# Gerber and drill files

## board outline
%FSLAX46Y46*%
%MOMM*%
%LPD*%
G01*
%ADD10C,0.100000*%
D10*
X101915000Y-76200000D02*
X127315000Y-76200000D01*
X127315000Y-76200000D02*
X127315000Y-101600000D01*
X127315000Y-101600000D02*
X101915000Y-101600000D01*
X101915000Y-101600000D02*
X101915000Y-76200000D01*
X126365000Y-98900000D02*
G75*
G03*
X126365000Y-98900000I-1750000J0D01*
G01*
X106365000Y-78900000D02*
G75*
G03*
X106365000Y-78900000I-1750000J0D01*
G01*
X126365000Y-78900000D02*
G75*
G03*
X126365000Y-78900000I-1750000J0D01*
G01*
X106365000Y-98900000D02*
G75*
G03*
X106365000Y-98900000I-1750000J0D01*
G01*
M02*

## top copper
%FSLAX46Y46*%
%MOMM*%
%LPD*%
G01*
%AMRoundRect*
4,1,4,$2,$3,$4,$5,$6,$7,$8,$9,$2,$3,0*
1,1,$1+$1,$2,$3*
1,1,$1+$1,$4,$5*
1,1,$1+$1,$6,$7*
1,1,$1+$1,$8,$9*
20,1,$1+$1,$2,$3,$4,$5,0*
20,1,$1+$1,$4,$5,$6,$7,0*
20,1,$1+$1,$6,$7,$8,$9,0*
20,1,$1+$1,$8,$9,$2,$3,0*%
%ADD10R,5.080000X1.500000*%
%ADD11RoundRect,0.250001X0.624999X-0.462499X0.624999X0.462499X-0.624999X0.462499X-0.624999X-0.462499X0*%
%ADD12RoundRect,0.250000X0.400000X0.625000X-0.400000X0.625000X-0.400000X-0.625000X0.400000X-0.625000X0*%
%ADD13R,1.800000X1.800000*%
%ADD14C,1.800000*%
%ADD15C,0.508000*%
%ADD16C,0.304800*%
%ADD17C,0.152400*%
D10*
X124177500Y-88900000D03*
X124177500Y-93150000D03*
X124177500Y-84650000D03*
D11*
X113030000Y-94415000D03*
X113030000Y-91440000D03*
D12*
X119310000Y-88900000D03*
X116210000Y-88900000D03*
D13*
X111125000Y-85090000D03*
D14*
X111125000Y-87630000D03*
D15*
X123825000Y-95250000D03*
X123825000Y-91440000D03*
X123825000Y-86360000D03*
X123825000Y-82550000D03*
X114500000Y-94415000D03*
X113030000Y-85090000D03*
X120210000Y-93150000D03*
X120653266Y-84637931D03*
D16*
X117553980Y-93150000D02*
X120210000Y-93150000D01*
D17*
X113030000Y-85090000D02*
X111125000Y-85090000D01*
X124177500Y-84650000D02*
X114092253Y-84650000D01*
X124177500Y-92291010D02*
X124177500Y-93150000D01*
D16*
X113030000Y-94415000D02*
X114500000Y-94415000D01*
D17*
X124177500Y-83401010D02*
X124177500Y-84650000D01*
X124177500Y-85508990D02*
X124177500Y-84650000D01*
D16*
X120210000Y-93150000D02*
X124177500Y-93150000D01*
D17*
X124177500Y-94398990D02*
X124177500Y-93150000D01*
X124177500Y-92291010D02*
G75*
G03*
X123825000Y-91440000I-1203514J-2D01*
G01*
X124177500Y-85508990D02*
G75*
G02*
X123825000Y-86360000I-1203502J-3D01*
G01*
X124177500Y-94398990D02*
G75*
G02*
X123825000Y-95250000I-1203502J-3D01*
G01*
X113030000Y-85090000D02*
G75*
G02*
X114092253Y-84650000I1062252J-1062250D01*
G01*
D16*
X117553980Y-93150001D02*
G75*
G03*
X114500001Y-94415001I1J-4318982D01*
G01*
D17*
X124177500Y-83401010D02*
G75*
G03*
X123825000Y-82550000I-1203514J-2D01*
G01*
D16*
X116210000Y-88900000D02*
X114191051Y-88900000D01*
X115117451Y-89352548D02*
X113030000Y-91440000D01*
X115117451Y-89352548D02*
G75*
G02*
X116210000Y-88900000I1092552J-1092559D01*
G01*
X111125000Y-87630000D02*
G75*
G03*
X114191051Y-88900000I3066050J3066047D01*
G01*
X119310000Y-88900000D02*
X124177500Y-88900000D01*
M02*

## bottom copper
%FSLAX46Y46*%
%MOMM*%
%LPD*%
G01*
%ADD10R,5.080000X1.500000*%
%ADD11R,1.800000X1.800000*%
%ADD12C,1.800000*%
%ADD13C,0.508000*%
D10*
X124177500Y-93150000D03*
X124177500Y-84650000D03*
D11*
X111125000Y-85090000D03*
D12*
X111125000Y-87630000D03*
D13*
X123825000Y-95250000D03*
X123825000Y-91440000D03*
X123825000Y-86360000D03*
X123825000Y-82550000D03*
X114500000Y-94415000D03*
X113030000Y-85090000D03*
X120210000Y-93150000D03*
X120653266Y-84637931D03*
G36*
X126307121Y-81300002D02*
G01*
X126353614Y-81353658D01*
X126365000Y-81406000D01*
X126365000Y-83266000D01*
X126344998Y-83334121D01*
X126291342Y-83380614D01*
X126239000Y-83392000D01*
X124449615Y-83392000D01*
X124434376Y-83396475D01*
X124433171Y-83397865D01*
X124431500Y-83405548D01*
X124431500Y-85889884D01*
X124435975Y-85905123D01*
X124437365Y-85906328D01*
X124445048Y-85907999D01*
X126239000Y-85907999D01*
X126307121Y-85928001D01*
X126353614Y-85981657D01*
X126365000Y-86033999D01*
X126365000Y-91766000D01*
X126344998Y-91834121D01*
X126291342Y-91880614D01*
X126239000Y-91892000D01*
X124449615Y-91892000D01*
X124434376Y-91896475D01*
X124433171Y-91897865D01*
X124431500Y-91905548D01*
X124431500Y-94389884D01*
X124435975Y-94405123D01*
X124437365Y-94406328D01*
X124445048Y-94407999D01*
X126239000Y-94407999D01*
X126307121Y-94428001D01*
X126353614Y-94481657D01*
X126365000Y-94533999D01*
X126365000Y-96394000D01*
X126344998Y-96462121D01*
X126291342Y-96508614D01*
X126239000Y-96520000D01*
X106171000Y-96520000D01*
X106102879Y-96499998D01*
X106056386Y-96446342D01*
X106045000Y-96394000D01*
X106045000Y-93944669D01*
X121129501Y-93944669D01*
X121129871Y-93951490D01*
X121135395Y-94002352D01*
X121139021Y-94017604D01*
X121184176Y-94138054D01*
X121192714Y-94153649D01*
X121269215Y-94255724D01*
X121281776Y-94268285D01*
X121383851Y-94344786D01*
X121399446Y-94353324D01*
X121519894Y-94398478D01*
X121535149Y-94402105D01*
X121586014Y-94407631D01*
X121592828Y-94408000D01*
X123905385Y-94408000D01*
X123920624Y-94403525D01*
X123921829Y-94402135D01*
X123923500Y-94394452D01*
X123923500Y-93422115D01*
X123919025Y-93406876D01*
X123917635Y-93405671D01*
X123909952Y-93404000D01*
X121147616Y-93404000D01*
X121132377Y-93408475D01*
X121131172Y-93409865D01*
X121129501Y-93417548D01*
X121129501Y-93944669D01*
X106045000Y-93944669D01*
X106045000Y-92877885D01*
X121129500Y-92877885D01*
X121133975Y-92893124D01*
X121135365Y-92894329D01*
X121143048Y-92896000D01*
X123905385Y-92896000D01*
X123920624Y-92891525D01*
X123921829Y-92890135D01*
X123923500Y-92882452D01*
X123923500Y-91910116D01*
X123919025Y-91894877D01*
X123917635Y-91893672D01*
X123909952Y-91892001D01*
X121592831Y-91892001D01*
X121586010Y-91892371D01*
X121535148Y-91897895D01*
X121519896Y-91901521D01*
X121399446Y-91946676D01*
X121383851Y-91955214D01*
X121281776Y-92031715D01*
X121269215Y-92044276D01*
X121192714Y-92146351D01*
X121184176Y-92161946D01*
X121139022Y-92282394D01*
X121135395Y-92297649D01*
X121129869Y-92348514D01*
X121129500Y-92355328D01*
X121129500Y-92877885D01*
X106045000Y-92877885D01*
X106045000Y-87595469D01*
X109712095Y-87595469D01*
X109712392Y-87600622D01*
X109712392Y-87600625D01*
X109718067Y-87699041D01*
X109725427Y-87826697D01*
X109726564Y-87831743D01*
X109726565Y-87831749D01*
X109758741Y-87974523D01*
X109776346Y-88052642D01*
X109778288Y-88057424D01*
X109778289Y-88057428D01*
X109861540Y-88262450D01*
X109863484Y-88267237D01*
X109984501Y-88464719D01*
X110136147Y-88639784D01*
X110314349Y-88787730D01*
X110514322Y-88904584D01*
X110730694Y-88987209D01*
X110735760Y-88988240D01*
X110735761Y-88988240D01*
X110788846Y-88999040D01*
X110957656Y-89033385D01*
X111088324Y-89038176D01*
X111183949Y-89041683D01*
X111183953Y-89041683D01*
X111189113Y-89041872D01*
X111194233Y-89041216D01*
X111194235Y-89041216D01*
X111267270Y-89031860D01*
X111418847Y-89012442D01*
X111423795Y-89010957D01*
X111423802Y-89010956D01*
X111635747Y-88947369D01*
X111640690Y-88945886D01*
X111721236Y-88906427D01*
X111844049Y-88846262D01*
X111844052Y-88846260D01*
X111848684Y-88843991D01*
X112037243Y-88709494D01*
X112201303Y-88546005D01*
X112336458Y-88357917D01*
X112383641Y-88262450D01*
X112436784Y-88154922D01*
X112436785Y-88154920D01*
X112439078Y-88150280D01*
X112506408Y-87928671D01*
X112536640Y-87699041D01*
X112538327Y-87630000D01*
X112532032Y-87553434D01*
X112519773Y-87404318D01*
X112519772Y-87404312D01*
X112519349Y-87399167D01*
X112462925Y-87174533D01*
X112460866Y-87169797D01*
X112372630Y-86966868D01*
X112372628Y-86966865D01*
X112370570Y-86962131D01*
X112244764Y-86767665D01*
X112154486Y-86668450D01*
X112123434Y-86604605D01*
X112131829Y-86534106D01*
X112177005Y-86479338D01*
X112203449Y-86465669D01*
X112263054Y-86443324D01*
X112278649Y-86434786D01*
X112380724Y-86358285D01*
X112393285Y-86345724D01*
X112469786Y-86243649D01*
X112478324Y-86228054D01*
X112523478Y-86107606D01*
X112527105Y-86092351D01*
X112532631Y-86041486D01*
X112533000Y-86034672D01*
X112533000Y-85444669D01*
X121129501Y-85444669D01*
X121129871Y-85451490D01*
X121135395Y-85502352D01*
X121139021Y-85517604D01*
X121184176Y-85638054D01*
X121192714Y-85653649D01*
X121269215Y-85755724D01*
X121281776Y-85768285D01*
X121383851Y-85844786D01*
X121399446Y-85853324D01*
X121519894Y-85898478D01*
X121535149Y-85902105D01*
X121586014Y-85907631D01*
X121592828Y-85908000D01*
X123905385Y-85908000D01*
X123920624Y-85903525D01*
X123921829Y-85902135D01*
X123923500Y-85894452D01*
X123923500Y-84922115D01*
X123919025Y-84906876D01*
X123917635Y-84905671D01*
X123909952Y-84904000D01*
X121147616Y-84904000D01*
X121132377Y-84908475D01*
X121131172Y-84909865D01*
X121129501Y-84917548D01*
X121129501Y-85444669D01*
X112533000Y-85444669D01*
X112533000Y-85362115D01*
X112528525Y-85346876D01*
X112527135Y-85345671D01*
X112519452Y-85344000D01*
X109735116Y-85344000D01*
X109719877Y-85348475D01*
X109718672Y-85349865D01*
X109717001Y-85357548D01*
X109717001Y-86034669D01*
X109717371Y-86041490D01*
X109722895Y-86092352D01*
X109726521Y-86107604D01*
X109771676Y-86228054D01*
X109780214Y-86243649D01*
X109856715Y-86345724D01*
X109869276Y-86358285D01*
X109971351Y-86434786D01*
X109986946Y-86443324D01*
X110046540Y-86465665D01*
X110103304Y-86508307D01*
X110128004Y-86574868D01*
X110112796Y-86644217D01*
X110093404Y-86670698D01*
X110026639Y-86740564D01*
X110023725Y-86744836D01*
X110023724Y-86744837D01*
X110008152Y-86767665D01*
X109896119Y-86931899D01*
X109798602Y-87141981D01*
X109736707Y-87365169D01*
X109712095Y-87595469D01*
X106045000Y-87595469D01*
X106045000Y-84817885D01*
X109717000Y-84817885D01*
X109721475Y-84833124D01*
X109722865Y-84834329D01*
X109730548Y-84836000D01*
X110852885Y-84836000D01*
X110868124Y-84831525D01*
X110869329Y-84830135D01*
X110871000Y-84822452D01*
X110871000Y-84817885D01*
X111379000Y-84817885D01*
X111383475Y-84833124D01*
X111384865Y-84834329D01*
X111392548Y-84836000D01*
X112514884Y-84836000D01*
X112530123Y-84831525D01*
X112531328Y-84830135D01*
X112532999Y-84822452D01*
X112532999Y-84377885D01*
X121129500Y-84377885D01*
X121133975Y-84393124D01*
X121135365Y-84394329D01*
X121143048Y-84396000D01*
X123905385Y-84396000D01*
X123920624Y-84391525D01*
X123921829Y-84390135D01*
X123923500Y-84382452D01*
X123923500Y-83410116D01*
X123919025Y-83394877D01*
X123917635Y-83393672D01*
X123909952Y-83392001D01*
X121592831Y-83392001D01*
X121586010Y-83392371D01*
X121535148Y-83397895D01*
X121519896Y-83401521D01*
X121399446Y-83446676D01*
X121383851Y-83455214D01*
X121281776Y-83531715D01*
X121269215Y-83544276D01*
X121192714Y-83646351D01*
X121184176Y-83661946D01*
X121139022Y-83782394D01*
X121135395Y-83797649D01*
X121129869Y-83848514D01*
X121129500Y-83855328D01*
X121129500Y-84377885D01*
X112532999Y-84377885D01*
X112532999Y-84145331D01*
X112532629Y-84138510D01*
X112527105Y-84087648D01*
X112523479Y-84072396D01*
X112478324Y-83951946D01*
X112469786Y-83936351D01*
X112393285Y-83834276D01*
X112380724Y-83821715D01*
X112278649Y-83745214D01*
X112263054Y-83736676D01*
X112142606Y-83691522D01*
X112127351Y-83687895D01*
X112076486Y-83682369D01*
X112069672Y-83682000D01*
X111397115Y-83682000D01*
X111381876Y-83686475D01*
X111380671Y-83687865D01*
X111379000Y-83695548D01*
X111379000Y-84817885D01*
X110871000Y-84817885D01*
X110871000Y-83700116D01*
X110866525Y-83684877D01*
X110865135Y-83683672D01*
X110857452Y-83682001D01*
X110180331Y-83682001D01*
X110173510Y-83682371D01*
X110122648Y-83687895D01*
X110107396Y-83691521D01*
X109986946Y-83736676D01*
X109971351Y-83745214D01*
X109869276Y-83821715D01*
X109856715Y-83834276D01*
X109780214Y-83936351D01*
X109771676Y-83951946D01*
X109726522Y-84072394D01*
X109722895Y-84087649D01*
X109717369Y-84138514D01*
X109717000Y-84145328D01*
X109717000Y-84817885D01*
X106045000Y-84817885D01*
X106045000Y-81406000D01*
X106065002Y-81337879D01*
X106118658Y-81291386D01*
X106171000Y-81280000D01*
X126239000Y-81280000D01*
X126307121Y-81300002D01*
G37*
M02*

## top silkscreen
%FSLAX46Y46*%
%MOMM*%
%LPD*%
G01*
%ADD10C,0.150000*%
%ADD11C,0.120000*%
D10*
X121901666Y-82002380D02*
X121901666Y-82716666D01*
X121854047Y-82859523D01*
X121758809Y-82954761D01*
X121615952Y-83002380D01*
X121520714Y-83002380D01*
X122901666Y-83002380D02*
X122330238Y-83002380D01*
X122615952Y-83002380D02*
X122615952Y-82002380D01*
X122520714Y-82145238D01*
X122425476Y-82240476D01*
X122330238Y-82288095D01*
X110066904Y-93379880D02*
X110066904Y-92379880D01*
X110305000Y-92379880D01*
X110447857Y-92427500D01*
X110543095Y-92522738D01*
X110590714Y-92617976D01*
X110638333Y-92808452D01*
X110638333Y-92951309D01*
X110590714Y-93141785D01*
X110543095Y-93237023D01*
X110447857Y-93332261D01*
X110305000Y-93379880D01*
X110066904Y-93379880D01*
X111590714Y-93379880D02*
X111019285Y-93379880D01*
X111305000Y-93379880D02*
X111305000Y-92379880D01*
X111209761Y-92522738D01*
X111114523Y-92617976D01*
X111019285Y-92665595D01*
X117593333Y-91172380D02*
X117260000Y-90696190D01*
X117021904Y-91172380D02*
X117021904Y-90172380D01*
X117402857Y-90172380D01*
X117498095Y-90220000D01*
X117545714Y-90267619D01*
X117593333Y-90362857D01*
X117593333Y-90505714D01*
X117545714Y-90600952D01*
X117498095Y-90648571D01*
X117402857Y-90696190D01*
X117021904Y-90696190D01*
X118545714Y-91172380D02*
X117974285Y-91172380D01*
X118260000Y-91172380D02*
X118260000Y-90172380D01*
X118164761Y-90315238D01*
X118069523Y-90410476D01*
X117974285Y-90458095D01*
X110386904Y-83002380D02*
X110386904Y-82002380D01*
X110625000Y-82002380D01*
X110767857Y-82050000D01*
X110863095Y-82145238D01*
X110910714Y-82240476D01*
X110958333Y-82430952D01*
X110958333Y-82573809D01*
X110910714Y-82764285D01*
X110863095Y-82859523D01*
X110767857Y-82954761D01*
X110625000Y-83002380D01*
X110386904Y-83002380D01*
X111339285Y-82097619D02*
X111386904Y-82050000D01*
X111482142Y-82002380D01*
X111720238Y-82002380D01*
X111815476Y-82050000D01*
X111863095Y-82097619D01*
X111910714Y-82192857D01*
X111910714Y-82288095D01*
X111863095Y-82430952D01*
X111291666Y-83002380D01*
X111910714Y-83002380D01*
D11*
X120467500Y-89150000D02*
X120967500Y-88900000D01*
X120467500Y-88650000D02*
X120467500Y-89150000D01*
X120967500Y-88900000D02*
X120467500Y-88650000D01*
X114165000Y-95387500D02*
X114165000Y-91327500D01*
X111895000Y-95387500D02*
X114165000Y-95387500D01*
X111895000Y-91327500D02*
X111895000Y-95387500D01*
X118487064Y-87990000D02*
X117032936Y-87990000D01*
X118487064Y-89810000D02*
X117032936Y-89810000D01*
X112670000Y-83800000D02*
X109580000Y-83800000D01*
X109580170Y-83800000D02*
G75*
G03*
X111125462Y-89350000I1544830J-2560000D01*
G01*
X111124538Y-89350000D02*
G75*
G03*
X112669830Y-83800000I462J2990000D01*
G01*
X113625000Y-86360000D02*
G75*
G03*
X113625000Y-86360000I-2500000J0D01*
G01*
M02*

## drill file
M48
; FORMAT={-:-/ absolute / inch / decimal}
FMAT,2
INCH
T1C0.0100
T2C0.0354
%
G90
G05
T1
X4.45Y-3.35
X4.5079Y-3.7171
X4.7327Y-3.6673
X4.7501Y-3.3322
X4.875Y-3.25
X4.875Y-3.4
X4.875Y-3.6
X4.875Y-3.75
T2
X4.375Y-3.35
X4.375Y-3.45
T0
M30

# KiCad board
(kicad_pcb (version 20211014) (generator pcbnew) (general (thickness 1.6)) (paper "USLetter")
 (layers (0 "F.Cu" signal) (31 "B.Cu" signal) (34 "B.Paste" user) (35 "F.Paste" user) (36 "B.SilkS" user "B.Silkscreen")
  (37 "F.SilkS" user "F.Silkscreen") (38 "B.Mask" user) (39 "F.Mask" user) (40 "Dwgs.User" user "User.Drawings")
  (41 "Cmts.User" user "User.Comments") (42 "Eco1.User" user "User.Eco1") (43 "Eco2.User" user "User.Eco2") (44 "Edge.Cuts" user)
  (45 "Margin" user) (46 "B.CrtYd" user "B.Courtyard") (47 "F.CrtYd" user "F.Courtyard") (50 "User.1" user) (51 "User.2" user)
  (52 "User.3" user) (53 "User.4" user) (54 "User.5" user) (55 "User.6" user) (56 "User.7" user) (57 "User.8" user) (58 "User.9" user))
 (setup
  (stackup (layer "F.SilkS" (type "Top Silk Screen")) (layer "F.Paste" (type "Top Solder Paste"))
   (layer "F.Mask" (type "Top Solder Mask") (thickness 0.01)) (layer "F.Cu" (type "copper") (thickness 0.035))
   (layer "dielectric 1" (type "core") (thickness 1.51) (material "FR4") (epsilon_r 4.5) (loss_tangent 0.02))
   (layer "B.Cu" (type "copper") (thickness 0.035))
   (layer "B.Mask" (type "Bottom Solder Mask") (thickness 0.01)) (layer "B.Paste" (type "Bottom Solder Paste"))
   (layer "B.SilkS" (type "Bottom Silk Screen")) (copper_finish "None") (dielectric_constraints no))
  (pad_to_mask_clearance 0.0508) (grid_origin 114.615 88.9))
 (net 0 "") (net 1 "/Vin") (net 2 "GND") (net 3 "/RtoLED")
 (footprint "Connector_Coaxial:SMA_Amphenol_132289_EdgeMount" (layer "F.Cu") (at 124.1775 88.9)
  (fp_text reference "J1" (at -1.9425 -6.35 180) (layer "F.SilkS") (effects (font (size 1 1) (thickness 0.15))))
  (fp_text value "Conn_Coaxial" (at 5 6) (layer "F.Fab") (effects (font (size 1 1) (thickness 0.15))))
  (fp_line (start -3.71 0.25) (end -3.21 0) (layer "F.SilkS") (width 0.12))
  (fp_line (start -3.71 -0.25) (end -3.71 0.25) (layer "F.SilkS") (width 0.12))
  (fp_line (start -3.21 0) (end -3.71 -0.25) (layer "F.SilkS") (width 0.12))
  (pad "1" smd rect (at 0 0 90) (size 1.5 5.08) (layers "F.Cu" "F.Paste" "F.Mask") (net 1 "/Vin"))
  (pad "2" smd rect (at 0 4.25 90) (size 1.5 5.08) (layers "F.Cu" "F.Paste" "F.Mask") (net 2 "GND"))
  (pad "2" smd rect (at 0 4.25 90) (size 1.5 5.08) (layers "B.Cu" "B.Paste" "B.Mask") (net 2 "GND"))
  (pad "2" smd rect (at 0 -4.25 90) (size 1.5 5.08) (layers "B.Cu" "B.Paste" "B.Mask") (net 2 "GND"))
  (pad "2" smd rect (at 0 -4.25 90) (size 1.5 5.08) (layers "F.Cu" "F.Paste" "F.Mask") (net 2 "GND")))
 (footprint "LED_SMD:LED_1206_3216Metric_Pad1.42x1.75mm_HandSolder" (layer "F.Cu") (at 113.03 92.9275 90)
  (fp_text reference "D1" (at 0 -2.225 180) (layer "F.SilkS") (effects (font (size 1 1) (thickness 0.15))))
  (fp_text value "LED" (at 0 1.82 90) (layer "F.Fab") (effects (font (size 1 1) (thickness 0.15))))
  (fp_line (start -2.46 1.135) (end 1.6 1.135) (layer "F.SilkS") (width 0.12))
  (fp_line (start -2.46 -1.135) (end -2.46 1.135) (layer "F.SilkS") (width 0.12))
  (fp_line (start 1.6 -1.135) (end -2.46 -1.135) (layer "F.SilkS") (width 0.12))
  (pad "1" smd roundrect (at -1.4875 0 90) (size 1.425 1.75) (layers "F.Cu" "F.Paste" "F.Mask") (roundrect_rratio 0.1754392982)
   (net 2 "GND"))
  (pad "2" smd roundrect (at 1.4875 0 90) (size 1.425 1.75) (layers "F.Cu" "F.Paste" "F.Mask") (roundrect_rratio 0.1754392982)
   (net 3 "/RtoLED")))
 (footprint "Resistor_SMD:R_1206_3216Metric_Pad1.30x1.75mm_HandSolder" (layer "F.Cu") (at 117.76 88.9 180)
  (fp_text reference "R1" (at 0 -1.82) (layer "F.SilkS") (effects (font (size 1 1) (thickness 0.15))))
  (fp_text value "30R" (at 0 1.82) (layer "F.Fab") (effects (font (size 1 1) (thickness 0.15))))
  (fp_line (start -0.727064 0.91) (end 0.727064 0.91) (layer "F.SilkS") (width 0.12))
  (fp_line (start -0.727064 -0.91) (end 0.727064 -0.91) (layer "F.SilkS") (width 0.12))
  (pad "1" smd roundrect (at -1.55 0 180) (size 1.3 1.75) (layers "F.Cu" "F.Paste" "F.Mask") (roundrect_rratio 0.1923076923) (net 1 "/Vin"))
  (pad "2" smd roundrect (at 1.55 0 180) (size 1.3 1.75) (layers "F.Cu" "F.Paste" "F.Mask") (roundrect_rratio 0.1923076923)
   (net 3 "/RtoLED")))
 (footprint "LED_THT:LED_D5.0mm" (layer "F.Cu") (at 111.125 85.09 -90)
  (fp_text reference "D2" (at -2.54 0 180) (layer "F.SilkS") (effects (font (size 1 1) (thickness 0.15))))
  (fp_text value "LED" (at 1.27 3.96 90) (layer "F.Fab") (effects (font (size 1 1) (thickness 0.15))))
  (fp_line (start -1.29 -1.545) (end -1.29 1.545) (layer "F.SilkS") (width 0.12))
  (fp_arc (start 4.26 -0.000462) (mid 2.072002 2.880433) (end -1.29 1.54483) (layer "F.SilkS") (width 0.12))
  (fp_arc (start -1.29 -1.54483) (mid 2.072002 -2.880433) (end 4.26 0.000462) (layer "F.SilkS") (width 0.12))
  (fp_circle (center 1.27 0) (end 3.77 0) (layer "F.SilkS") (width 0.12) (fill none))
  (pad "1" thru_hole rect (at 0 0 270) (size 1.8 1.8) (drill 0.9) (layers *.Cu *.Mask) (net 2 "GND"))
  (pad "2" thru_hole circle (at 2.54 0 270) (size 1.8 1.8) (drill 0.9) (layers *.Cu *.Mask) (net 3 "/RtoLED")))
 (gr_rect (start 101.915 76.2) (end 127.315 101.6) (layer "Edge.Cuts") (width 0.1) (fill none))
 (gr_circle (center 124.615 98.9) (end 126.365 98.9) (layer "Edge.Cuts") (width 0.1) (fill none))
 (gr_circle (center 104.615 78.9) (end 106.365 78.9) (layer "Edge.Cuts") (width 0.1) (fill none))
 (gr_circle (center 124.615 78.9) (end 126.365 78.9) (layer "Edge.Cuts") (width 0.1) (fill none))
 (gr_circle (center 104.615 98.9) (end 106.365 98.9) (layer "Edge.Cuts") (width 0.1) (fill none))
 (segment (start 117.55398 93.15) (end 120.21 93.15) (width 0.3048) (layer "F.Cu") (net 2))
 (segment (start 113.03 85.09) (end 111.125 85.09) (width 0.1524) (layer "F.Cu") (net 2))
 (segment (start 124.1775 84.65) (end 114.092253 84.65) (width 0.1524) (layer "F.Cu") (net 2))
 (segment (start 124.1775 92.29101) (end 124.1775 93.15) (width 0.1524) (layer "F.Cu") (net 2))
 (segment (start 113.03 94.415) (end 114.5 94.415) (width 0.3048) (layer "F.Cu") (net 2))
 (segment (start 124.1775 83.40101) (end 124.1775 84.65) (width 0.1524) (layer "F.Cu") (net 2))
 (segment (start 124.1775 85.50899) (end 124.1775 84.65) (width 0.1524) (layer "F.Cu") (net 2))
 (segment (start 120.21 93.15) (end 124.1775 93.15) (width 0.3048) (layer "F.Cu") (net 2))
 (segment (start 124.1775 94.39899) (end 124.1775 93.15) (width 0.1524) (layer "F.Cu") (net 2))
 (via (at 123.825 95.25) (size 0.508) (drill 0.254) (layers "F.Cu" "B.Cu") (free) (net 2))
 (via (at 123.825 91.44) (size 0.508) (drill 0.254) (layers "F.Cu" "B.Cu") (free) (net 2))
 (via (at 123.825 86.36) (size 0.508) (drill 0.254) (layers "F.Cu" "B.Cu") (free) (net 2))
 (via (at 123.825 82.55) (size 0.508) (drill 0.254) (layers "F.Cu" "B.Cu") (free) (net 2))
 (via (at 114.5 94.415) (size 0.508) (drill 0.254) (layers "F.Cu" "B.Cu") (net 2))
 (via (at 113.03 85.09) (size 0.508) (drill 0.254) (layers "F.Cu" "B.Cu") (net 2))
 (via (at 120.21 93.15) (size 0.508) (drill 0.254) (layers "F.Cu" "B.Cu") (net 2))
 (via (at 120.653266 84.637931) (size 0.508) (drill 0.254) (layers "F.Cu" "B.Cu") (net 2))
 (arc (start 123.825 91.44) (mid 124.085888 91.830447) (end 124.1775 92.29101) (width 0.1524) (layer "F.Cu") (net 2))
 (arc (start 123.825 86.36) (mid 124.085889 85.969553) (end 124.1775 85.50899) (width 0.1524) (layer "F.Cu") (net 2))
 (arc (start 123.825 95.25) (mid 124.085889 94.859553) (end 124.1775 94.39899) (width 0.1524) (layer "F.Cu") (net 2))
 (arc (start 114.092253 84.65) (mid 113.517366 84.764352) (end 113.03 85.09) (width 0.1524) (layer "F.Cu") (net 2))
 (arc (start 114.5 94.415) (mid 115.901178 93.478763) (end 117.55398 93.15) (width 0.3048) (layer "F.Cu") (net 2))
 (arc (start 123.825 82.55) (mid 124.085888 82.940447) (end 124.1775 83.40101) (width 0.1524) (layer "F.Cu") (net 2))
 (segment (start 116.21 88.9) (end 114.191051 88.9) (width 0.3048) (layer "F.Cu") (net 3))
 (segment (start 115.117451 89.352548) (end 113.03 91.44) (width 0.3048) (layer "F.Cu") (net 3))
 (arc (start 116.21 88.9) (mid 115.618717 89.017614) (end 115.117451 89.352548) (width 0.3048) (layer "F.Cu") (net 3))
 (arc (start 114.191051 88.9) (mid 112.531716 88.569938) (end 111.125 87.63) (width 0.3048) (layer "F.Cu") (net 3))
 (segment (start 119.31 88.9) (end 124.1775 88.9) (width 0.3048) (layer "F.Cu") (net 1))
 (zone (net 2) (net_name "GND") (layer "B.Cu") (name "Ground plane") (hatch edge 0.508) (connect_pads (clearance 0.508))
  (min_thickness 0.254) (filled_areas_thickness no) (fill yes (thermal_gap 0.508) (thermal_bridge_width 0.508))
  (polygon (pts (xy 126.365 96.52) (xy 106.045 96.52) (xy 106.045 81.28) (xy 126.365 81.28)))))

